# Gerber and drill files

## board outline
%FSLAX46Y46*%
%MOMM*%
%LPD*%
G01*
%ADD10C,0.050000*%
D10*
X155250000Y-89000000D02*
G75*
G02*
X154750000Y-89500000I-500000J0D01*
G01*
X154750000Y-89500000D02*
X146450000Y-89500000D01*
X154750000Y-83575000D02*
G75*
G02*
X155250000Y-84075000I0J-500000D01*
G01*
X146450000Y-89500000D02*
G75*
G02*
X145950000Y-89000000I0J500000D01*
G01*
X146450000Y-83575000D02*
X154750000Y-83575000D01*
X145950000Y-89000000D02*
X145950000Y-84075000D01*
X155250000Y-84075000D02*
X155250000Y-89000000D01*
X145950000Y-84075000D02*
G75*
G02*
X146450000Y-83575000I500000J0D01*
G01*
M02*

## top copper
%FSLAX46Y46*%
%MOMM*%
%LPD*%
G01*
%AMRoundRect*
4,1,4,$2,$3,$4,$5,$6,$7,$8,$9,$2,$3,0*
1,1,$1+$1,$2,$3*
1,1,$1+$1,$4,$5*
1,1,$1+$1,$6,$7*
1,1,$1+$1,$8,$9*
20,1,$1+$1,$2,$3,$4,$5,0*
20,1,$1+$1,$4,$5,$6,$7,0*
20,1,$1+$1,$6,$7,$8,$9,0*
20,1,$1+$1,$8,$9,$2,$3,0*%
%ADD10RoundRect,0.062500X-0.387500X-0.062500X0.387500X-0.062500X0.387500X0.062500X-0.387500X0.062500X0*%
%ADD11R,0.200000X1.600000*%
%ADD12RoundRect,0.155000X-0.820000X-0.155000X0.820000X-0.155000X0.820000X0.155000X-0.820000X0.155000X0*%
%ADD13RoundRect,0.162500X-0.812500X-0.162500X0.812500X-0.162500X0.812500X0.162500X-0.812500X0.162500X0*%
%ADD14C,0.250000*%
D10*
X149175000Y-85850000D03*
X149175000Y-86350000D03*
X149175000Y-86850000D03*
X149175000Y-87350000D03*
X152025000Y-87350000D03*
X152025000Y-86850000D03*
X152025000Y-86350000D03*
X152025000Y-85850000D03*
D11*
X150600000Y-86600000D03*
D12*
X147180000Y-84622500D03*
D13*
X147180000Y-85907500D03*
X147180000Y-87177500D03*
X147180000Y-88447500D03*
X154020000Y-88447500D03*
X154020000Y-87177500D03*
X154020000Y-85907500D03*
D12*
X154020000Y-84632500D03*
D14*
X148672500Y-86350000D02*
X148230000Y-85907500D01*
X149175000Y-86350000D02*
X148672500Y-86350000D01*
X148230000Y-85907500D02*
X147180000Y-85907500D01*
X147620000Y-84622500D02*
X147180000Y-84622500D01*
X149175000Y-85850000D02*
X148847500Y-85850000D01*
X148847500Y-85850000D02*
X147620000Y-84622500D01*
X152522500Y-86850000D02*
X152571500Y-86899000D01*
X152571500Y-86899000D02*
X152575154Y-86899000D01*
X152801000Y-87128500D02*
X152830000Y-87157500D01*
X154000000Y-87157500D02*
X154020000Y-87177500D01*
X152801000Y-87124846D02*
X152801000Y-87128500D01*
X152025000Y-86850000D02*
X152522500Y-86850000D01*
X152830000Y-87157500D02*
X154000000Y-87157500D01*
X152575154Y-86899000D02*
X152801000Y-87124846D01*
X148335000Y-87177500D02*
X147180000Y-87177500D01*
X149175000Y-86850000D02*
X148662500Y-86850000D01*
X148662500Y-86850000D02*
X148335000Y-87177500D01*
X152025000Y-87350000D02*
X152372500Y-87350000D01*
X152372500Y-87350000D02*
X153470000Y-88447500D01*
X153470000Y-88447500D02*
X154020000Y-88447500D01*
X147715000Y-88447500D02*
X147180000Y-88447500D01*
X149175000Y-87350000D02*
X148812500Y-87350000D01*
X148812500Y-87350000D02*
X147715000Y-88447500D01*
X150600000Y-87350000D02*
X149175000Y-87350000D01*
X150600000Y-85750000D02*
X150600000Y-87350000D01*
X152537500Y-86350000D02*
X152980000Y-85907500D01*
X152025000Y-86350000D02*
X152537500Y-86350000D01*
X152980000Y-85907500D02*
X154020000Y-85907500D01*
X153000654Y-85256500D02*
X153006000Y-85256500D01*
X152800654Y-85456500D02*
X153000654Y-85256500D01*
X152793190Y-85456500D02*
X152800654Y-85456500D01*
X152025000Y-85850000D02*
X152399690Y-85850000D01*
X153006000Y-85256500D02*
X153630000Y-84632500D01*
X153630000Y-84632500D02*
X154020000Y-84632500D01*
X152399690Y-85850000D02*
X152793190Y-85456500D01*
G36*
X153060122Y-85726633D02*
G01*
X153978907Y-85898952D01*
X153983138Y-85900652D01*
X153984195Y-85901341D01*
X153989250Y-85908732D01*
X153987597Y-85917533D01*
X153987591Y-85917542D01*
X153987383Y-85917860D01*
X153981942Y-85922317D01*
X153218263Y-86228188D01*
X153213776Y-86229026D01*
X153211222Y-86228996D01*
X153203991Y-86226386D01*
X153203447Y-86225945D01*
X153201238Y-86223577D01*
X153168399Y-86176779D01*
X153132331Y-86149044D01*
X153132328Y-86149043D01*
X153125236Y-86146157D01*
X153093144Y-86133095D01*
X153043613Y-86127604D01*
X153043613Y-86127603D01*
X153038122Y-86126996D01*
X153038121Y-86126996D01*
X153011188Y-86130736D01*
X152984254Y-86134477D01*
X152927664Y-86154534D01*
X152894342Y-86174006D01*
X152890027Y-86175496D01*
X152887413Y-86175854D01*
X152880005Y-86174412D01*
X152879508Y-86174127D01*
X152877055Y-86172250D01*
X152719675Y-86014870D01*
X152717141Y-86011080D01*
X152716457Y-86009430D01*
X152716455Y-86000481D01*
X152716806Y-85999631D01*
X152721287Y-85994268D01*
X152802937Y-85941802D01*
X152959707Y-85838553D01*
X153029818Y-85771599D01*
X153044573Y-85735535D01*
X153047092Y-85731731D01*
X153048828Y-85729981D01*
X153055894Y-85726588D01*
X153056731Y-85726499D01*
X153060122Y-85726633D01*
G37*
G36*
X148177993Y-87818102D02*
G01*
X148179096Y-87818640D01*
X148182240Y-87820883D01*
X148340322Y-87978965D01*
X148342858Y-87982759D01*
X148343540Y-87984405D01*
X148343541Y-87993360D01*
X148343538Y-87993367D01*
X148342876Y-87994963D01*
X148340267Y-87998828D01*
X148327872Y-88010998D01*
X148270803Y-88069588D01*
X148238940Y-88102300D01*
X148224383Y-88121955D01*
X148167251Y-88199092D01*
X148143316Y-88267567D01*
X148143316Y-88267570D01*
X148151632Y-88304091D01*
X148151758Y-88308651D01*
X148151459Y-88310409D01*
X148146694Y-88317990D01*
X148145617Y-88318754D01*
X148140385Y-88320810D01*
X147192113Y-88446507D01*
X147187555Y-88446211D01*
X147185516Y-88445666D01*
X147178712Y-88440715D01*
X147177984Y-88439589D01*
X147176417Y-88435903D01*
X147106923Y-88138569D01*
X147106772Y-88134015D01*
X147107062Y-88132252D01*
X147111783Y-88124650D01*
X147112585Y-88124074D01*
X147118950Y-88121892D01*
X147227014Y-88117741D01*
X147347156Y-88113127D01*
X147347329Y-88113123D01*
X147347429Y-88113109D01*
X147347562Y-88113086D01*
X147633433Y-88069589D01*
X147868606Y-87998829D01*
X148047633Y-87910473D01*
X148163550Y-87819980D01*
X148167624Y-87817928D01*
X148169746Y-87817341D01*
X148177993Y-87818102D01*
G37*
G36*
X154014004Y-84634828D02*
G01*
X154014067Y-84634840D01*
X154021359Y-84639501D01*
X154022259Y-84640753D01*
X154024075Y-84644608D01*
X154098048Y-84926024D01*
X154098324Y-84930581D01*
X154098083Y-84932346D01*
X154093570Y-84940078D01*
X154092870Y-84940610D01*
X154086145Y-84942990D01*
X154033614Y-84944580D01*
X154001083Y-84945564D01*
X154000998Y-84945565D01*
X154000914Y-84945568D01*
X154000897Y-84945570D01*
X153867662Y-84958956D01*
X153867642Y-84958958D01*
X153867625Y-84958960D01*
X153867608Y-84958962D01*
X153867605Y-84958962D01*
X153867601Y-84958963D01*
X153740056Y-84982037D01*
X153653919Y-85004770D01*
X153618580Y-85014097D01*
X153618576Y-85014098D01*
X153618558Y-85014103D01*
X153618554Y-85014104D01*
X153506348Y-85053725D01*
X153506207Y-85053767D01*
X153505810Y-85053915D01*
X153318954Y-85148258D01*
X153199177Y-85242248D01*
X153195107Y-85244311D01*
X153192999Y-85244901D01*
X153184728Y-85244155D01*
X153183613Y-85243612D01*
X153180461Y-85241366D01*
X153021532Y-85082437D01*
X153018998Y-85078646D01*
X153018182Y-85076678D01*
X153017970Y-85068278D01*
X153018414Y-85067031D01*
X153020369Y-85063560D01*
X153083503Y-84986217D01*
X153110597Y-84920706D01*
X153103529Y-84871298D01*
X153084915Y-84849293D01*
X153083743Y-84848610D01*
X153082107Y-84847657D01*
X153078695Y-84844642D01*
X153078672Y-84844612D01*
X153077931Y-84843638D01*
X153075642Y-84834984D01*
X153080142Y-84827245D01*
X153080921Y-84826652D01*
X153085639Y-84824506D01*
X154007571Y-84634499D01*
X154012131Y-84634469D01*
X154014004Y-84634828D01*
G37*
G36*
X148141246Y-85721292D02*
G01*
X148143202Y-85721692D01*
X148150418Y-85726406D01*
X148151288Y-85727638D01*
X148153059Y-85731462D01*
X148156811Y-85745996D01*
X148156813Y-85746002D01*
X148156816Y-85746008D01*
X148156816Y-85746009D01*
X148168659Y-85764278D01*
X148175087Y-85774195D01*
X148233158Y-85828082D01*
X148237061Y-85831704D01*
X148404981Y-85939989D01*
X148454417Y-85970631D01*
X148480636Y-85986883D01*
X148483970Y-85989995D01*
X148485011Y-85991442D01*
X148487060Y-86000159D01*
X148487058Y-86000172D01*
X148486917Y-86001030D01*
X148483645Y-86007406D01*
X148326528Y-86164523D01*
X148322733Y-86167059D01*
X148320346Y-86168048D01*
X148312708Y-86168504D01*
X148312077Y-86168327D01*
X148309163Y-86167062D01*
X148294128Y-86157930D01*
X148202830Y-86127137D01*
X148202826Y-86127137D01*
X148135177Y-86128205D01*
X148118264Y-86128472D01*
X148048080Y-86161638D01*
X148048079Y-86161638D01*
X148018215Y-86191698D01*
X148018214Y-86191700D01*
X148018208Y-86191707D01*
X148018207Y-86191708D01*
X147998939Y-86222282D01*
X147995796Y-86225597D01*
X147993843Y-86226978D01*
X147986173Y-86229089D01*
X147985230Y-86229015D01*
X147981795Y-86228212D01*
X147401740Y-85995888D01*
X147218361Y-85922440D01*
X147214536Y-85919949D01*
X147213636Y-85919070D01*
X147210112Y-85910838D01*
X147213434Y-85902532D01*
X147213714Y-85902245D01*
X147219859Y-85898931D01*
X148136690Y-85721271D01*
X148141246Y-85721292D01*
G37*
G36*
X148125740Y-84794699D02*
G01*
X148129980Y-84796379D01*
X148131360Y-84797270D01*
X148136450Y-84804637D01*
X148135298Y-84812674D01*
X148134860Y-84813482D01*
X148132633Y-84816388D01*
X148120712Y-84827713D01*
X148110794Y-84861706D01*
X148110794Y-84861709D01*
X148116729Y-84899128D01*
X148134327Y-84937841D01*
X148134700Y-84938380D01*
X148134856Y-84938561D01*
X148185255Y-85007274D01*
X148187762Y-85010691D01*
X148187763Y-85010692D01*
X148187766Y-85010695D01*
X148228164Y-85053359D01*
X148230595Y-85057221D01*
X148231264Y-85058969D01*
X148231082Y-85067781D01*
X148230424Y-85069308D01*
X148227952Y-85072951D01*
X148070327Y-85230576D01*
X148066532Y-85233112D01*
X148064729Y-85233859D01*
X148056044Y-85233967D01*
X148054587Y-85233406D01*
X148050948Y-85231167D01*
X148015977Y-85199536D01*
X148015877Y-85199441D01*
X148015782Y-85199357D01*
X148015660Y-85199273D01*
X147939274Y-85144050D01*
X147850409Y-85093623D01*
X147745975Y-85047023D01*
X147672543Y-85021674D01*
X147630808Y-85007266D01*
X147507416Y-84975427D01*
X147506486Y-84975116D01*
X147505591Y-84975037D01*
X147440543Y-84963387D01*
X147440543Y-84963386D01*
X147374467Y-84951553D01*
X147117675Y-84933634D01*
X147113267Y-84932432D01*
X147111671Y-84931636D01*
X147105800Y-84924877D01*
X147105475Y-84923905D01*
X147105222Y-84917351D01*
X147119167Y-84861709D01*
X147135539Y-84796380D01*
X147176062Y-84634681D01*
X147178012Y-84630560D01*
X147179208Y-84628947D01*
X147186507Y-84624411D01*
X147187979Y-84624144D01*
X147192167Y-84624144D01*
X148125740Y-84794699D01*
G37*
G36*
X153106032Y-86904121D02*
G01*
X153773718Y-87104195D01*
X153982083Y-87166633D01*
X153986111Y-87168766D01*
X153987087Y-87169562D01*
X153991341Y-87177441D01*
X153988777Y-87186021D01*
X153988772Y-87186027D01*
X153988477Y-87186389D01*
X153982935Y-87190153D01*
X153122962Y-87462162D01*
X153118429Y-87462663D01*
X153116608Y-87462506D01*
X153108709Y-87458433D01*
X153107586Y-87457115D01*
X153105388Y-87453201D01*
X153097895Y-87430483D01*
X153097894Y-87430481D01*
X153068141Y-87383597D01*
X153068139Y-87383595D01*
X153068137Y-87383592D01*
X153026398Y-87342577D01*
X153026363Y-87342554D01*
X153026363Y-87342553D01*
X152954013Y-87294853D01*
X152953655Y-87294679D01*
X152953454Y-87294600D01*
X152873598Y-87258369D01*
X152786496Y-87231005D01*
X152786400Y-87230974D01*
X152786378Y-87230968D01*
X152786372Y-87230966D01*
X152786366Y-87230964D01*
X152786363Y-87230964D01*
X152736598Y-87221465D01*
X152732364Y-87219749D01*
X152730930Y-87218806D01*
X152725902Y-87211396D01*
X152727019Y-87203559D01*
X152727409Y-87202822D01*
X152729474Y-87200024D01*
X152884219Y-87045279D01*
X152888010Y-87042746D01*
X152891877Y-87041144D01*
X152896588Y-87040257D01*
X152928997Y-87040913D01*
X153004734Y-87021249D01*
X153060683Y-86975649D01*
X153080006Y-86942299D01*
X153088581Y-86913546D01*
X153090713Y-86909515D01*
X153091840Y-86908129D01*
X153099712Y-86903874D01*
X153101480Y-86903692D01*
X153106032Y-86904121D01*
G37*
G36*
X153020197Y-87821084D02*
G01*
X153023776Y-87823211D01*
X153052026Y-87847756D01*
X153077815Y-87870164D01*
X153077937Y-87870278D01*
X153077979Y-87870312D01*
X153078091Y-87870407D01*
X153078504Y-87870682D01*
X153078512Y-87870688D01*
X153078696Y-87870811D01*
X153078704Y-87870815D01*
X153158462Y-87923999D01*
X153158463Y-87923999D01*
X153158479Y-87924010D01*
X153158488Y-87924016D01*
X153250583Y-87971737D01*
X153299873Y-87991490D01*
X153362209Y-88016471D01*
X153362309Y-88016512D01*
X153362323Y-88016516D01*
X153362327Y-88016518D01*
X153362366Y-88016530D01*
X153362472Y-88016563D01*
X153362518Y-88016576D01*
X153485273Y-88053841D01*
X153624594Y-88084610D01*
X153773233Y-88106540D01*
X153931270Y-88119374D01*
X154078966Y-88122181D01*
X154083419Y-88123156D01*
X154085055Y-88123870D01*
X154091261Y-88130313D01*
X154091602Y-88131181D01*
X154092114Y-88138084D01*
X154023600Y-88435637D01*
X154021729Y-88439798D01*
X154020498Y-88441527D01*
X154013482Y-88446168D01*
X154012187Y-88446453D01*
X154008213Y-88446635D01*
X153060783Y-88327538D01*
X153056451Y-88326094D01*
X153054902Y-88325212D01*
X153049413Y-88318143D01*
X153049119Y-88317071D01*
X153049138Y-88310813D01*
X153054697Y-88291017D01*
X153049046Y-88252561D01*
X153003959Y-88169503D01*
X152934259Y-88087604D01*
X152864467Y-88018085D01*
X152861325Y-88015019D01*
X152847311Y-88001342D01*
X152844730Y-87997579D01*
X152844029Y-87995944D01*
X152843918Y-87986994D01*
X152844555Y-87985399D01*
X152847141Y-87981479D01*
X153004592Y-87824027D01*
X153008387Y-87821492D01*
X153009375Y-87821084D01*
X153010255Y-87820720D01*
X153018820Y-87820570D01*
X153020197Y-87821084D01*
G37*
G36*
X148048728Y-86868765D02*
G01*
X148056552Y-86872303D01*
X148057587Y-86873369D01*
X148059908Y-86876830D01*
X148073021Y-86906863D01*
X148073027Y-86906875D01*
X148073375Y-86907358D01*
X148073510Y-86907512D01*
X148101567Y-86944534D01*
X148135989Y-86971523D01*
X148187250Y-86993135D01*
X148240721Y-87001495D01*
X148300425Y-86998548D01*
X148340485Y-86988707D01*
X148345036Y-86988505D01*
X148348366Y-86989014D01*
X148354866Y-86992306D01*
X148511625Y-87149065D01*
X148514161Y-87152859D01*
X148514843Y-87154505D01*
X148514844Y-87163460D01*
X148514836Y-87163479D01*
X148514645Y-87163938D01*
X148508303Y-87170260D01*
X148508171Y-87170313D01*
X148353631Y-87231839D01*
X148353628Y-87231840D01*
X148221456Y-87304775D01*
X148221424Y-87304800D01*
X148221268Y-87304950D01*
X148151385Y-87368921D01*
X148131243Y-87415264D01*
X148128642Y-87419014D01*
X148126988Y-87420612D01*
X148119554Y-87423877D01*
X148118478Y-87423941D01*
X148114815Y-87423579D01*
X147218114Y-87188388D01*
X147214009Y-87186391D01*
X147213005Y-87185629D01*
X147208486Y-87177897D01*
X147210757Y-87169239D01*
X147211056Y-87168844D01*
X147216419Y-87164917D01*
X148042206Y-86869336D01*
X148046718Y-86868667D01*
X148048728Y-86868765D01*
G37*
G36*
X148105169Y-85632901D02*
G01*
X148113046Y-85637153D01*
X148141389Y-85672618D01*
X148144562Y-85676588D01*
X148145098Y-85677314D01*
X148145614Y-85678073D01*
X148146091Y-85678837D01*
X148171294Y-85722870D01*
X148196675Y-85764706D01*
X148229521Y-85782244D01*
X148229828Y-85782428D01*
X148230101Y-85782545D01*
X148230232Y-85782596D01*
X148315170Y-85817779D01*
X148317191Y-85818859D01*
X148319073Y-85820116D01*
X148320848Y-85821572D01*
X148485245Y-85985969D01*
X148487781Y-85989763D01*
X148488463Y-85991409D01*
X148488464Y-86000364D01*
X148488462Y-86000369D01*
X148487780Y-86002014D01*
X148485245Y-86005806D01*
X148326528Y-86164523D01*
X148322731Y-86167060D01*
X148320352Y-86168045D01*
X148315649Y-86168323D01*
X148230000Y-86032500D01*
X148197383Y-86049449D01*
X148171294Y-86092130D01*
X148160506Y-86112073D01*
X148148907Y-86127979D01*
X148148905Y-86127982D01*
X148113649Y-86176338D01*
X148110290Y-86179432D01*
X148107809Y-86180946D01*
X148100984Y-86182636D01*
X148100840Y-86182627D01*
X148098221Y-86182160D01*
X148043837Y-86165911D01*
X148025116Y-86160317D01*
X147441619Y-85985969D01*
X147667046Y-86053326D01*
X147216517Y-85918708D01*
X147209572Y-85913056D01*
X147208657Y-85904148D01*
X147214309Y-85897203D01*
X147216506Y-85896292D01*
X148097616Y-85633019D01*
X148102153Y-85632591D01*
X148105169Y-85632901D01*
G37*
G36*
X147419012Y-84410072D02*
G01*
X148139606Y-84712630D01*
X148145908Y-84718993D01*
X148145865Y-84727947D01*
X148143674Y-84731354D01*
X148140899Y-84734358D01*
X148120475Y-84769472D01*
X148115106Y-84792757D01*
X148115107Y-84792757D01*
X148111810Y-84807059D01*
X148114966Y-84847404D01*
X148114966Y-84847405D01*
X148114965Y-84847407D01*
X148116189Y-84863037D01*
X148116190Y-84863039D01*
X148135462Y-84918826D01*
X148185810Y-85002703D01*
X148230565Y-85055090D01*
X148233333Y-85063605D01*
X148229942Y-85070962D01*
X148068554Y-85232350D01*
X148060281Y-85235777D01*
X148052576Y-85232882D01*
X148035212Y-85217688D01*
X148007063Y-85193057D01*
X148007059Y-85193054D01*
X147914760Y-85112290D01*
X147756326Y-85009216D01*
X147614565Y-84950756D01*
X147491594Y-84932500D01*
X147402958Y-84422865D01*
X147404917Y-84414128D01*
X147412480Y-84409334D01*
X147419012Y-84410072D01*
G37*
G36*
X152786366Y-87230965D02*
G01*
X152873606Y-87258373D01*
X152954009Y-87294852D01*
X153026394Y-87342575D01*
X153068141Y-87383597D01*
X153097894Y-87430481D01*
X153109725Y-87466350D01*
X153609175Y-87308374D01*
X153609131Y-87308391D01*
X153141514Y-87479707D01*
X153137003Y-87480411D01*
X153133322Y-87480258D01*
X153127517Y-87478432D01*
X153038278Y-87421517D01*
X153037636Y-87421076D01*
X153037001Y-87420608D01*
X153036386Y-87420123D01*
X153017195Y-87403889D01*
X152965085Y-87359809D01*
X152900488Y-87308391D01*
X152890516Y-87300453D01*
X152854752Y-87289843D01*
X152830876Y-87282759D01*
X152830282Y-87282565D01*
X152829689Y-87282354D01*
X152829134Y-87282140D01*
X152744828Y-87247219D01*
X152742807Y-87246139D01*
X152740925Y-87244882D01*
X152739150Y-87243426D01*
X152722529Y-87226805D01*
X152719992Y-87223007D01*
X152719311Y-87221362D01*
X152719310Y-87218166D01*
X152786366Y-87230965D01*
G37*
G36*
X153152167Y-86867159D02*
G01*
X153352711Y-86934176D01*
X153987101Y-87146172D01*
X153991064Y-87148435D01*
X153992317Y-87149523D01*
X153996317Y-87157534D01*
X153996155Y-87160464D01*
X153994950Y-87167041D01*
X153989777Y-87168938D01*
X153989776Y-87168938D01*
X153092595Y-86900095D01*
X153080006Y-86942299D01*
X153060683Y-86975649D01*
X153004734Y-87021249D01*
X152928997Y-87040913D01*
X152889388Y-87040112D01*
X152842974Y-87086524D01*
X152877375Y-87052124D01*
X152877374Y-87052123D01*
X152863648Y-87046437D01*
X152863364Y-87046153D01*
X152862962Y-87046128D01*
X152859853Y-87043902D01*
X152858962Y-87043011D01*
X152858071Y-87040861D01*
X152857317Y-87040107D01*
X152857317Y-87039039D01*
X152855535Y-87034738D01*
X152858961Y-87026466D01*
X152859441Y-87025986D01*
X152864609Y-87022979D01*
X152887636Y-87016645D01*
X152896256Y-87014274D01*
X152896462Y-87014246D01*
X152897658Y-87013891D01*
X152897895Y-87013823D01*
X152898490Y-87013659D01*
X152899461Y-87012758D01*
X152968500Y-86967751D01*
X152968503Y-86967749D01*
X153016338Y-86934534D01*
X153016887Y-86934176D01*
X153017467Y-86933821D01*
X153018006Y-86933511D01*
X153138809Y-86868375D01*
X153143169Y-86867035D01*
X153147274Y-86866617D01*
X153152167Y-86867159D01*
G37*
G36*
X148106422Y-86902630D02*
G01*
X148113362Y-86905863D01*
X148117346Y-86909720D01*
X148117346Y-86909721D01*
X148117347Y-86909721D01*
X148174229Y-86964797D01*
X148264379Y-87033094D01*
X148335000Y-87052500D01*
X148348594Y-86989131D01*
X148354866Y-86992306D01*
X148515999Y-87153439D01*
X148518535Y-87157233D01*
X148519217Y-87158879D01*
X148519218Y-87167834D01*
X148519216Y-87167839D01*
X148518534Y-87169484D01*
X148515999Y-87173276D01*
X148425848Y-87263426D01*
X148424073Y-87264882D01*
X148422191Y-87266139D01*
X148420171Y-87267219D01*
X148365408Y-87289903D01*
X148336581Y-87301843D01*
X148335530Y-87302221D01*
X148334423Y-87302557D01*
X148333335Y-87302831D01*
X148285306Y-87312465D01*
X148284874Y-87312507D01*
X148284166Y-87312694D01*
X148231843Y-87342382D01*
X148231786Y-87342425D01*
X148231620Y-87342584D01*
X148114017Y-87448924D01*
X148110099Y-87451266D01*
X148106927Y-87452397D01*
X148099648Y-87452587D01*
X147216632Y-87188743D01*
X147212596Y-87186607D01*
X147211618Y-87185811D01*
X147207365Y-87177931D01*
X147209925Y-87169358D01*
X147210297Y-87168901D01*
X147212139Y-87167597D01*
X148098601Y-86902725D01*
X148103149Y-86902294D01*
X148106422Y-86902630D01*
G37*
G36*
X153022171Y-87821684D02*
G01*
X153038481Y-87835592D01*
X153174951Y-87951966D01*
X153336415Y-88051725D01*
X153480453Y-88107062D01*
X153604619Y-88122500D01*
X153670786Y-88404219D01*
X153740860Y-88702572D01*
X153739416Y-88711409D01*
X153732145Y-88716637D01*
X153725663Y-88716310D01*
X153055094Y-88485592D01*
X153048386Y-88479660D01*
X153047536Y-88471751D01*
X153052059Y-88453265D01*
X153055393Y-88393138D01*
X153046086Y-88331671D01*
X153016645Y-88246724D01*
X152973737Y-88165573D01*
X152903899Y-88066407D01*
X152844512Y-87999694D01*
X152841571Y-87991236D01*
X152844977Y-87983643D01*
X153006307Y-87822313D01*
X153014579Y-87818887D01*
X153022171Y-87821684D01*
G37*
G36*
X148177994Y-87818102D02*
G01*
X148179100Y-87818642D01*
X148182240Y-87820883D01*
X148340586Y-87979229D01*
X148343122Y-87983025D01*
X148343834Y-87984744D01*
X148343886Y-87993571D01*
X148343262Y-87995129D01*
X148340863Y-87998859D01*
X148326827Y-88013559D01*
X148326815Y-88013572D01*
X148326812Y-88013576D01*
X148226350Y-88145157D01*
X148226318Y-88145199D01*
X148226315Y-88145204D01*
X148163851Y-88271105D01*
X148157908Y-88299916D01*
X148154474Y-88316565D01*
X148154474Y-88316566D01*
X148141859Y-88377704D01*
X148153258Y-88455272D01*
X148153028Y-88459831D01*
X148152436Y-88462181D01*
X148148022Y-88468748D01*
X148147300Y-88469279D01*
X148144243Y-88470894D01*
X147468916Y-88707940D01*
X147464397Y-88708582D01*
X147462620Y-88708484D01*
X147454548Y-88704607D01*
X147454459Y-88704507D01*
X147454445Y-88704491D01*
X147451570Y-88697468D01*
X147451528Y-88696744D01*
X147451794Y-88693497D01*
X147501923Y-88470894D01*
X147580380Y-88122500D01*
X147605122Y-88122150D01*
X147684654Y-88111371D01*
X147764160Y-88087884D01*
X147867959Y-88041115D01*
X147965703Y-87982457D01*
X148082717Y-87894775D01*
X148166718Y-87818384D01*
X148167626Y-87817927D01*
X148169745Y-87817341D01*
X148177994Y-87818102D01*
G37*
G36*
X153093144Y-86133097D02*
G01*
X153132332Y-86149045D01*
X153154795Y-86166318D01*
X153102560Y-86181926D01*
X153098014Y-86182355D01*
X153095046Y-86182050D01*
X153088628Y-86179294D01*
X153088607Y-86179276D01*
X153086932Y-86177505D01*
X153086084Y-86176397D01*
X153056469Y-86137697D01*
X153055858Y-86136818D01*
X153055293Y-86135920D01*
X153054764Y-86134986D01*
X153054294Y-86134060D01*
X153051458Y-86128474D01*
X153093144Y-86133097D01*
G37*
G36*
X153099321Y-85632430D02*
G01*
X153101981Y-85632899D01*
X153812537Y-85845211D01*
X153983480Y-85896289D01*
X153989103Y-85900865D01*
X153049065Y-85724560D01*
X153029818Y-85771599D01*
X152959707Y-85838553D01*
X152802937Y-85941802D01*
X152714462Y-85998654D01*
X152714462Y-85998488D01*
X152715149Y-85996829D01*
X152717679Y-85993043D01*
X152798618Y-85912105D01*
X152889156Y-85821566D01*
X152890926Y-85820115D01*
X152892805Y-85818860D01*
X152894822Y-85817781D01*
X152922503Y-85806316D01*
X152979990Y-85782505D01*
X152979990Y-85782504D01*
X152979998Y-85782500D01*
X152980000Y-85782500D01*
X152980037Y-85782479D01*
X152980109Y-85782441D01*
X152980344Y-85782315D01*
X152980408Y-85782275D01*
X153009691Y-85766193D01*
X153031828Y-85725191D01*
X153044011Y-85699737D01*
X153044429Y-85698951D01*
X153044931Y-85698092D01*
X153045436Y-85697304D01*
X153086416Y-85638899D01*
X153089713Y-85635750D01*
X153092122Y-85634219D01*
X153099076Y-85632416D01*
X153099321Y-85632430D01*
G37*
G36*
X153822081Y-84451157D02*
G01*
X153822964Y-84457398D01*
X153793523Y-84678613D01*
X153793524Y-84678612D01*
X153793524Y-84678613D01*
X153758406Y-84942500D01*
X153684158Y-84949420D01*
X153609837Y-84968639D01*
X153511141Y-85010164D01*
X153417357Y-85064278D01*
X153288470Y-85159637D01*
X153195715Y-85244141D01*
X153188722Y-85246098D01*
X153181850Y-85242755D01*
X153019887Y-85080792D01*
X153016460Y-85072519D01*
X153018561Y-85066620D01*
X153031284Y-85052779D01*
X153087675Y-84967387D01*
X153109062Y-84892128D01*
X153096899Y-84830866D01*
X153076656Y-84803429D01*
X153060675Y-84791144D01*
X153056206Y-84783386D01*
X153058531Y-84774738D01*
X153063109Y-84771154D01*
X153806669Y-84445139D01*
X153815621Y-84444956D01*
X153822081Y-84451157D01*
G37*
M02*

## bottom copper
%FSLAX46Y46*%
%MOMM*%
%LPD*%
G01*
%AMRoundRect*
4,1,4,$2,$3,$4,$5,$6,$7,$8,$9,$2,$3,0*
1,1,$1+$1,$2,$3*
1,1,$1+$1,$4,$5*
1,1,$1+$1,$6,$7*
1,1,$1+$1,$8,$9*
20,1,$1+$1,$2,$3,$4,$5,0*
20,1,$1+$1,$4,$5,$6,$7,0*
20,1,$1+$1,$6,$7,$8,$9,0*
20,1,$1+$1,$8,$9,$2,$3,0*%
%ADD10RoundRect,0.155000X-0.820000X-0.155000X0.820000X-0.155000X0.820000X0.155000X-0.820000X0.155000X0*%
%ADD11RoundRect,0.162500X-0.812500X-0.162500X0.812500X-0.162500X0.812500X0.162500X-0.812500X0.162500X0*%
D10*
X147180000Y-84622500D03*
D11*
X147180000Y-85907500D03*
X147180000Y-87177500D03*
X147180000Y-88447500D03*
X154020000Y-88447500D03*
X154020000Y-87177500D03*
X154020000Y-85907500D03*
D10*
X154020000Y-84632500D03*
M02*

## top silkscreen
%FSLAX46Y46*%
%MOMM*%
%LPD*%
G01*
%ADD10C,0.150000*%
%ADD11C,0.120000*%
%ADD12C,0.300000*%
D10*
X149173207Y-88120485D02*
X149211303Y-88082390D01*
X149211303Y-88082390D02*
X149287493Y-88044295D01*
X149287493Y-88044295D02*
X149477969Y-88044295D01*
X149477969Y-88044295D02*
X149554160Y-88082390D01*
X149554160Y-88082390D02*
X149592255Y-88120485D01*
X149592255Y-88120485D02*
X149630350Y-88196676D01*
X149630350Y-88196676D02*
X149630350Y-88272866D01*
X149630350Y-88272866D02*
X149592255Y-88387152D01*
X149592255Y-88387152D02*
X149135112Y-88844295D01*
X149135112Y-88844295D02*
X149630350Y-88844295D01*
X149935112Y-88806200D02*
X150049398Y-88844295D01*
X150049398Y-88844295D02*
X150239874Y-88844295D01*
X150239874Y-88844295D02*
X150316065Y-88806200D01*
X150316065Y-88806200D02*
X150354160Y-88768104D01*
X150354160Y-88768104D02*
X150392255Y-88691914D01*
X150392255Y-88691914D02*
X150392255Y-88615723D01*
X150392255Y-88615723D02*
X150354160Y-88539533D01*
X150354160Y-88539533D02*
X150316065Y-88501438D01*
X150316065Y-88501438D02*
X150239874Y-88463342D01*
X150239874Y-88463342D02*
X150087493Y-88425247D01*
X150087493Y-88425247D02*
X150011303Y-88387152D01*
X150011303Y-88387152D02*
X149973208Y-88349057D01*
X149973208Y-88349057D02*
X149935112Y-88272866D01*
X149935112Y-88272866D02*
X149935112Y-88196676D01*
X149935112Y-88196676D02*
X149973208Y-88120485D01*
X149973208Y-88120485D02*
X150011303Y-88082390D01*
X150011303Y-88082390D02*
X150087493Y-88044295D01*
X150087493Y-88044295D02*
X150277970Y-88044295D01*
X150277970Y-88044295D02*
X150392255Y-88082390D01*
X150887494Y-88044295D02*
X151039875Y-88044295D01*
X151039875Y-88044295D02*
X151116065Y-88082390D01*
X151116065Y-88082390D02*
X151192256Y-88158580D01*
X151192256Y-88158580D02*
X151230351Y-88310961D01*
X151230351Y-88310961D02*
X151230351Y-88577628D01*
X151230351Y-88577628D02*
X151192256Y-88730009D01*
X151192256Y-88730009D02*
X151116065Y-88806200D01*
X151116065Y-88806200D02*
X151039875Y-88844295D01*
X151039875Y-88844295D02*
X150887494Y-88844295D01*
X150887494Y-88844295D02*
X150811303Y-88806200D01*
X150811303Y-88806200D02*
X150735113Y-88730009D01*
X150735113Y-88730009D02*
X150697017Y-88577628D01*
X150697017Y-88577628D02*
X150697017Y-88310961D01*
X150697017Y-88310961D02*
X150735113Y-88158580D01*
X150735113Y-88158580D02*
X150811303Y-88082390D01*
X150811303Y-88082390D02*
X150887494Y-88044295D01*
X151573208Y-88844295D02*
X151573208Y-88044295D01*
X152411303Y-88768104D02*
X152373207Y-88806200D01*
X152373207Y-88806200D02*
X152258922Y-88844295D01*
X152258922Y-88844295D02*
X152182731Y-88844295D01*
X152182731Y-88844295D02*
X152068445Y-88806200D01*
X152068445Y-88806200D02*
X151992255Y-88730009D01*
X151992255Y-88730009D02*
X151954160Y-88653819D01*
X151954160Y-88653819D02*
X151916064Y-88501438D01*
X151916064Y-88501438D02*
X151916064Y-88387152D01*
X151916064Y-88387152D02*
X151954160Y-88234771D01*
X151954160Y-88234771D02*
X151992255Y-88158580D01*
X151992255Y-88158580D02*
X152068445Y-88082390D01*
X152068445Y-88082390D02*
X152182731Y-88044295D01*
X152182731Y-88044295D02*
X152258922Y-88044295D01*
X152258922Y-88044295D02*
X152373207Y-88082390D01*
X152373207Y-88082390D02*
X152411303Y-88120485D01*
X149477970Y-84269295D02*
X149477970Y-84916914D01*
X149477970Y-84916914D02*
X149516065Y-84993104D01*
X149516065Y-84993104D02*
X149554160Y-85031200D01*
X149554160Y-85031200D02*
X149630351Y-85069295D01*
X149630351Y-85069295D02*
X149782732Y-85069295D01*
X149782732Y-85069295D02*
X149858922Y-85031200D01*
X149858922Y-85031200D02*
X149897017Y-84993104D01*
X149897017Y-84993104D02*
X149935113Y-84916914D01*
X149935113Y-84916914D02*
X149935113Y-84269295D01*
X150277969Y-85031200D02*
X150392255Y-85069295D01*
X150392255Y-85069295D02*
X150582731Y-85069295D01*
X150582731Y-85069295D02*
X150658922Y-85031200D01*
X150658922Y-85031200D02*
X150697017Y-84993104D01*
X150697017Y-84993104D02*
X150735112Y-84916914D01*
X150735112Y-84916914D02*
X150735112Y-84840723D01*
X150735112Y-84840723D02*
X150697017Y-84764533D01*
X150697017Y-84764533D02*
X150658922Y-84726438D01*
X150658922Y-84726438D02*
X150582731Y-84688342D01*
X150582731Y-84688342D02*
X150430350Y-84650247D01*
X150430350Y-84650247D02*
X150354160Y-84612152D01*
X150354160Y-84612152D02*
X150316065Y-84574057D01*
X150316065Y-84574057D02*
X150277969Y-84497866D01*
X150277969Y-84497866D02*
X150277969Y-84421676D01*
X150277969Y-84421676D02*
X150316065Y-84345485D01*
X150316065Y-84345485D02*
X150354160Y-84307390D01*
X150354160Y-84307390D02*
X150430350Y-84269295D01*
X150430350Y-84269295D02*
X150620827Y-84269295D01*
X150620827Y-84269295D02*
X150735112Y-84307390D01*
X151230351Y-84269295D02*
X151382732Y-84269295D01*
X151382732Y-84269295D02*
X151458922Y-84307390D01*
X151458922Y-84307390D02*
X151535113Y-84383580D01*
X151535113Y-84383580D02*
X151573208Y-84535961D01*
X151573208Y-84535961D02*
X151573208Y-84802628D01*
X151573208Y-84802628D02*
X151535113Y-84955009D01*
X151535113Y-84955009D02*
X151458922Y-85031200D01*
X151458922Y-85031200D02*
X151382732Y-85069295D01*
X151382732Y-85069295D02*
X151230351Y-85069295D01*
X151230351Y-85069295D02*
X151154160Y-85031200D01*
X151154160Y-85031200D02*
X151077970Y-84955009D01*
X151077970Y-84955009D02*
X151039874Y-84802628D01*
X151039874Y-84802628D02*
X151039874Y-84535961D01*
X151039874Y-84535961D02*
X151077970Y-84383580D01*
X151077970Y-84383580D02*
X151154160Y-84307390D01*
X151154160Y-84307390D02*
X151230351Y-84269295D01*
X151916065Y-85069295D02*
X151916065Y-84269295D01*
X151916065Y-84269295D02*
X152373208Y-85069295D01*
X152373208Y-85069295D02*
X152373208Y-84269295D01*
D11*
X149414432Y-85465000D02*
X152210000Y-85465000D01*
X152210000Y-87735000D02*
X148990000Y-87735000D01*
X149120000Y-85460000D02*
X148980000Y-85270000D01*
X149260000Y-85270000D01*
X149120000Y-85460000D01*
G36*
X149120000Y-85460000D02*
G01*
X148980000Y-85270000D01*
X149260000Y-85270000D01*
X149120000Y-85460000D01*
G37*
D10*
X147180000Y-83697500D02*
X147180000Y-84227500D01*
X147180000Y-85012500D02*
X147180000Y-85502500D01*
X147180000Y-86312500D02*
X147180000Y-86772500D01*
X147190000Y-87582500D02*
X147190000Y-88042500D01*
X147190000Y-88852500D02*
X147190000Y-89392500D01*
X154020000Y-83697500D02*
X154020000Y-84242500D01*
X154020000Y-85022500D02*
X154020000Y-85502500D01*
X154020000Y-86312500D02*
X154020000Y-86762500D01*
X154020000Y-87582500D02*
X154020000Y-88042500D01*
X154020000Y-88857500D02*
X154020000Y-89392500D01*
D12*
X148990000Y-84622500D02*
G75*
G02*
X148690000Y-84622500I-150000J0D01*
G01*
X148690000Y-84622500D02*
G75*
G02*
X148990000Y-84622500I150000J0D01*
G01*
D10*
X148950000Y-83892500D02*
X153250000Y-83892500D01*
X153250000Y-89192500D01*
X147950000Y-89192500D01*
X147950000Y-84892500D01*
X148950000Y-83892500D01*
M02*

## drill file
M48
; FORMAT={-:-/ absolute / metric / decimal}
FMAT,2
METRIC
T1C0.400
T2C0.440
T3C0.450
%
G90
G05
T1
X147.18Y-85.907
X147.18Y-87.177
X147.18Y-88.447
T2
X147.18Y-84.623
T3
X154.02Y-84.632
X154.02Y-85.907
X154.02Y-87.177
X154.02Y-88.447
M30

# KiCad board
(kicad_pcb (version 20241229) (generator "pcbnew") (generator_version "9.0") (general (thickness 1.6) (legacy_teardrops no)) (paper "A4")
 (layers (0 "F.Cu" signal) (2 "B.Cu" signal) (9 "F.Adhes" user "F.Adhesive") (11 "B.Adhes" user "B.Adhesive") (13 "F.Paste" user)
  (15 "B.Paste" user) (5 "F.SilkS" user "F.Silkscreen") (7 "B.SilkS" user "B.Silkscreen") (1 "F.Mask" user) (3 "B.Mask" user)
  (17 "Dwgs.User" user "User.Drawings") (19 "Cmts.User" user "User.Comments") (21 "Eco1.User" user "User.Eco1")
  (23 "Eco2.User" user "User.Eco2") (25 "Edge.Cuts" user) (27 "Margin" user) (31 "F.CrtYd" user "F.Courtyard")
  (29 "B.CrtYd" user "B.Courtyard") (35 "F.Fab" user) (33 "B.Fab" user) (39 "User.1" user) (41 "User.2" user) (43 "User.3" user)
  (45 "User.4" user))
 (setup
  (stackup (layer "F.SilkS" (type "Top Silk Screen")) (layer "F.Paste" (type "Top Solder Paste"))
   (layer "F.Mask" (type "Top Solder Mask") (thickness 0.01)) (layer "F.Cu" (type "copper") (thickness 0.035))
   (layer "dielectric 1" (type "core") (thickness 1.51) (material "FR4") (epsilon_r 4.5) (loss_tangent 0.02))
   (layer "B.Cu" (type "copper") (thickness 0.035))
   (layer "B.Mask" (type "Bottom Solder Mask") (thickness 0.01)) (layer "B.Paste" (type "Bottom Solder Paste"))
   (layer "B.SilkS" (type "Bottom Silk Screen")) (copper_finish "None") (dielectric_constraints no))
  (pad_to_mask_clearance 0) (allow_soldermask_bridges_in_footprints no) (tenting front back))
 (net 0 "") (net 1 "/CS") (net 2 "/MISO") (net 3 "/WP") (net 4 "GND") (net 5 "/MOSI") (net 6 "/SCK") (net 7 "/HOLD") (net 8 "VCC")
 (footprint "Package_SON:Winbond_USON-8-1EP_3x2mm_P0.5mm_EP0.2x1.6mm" (layer "F.Cu") (at 150.6 86.6)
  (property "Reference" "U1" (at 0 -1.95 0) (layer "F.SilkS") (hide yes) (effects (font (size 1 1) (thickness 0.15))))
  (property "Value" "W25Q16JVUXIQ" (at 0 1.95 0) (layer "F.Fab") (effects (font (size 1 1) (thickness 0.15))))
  (fp_line (start -1.185568 -1.135) (end 1.61 -1.135) (stroke (width 0.12) (type solid)) (layer "F.SilkS"))
  (fp_line (start 1.61 1.135) (end -1.61 1.135) (stroke (width 0.12) (type solid)) (layer "F.SilkS"))
  (fp_poly (pts (xy -1.48 -1.14) (xy -1.62 -1.33) (xy -1.34 -1.33)) (stroke (width 0.12) (type solid)) (fill yes) (layer "F.SilkS"))
  (pad "" smd roundrect (at 0 0) (size 0.16 1.29) (layers "F.Paste") (roundrect_rratio 0.25)
   (teardrops (best_length_ratio 0.5) (max_length 1) (best_width_ratio 1) (max_width 2) (curved_edges yes) (filter_ratio 0.9) (enabled yes)
    (allow_two_segments yes) (prefer_zone_connections yes)))
  (pad "1" smd roundrect (at -1.425 -0.75) (size 0.9 0.25) (layers "F.Cu" "F.Mask" "F.Paste") (roundrect_rratio 0.25) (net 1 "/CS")
   (teardrops (best_length_ratio 0.5) (max_length 1) (best_width_ratio 1) (max_width 2) (curved_edges yes) (filter_ratio 0.9) (enabled yes)
    (allow_two_segments yes) (prefer_zone_connections yes)))
  (pad "2" smd roundrect (at -1.425 -0.25) (size 0.9 0.25) (layers "F.Cu" "F.Mask" "F.Paste") (roundrect_rratio 0.25) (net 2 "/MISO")
   (teardrops (best_length_ratio 0.5) (max_length 1) (best_width_ratio 1) (max_width 2) (curved_edges yes) (filter_ratio 0.9) (enabled yes)
    (allow_two_segments yes) (prefer_zone_connections yes)))
  (pad "3" smd roundrect (at -1.425 0.25) (size 0.9 0.25) (layers "F.Cu" "F.Mask" "F.Paste") (roundrect_rratio 0.25) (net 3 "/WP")
   (teardrops (best_length_ratio 0.5) (max_length 1) (best_width_ratio 1) (max_width 2) (curved_edges yes) (filter_ratio 0.9) (enabled yes)
    (allow_two_segments yes) (prefer_zone_connections yes)))
  (pad "4" smd roundrect (at -1.425 0.75) (size 0.9 0.25) (layers "F.Cu" "F.Mask" "F.Paste") (roundrect_rratio 0.25) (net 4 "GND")
   (teardrops (best_length_ratio 0.5) (max_length 1) (best_width_ratio 1) (max_width 2) (curved_edges yes) (filter_ratio 0.9) (enabled yes)
    (allow_two_segments yes) (prefer_zone_connections yes)))
  (pad "5" smd roundrect (at 1.425 0.75) (size 0.9 0.25) (layers "F.Cu" "F.Mask" "F.Paste") (roundrect_rratio 0.25) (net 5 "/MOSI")
   (teardrops (best_length_ratio 0.5) (max_length 1) (best_width_ratio 1) (max_width 2) (curved_edges yes) (filter_ratio 0.9) (enabled yes)
    (allow_two_segments yes) (prefer_zone_connections yes)))
  (pad "6" smd roundrect (at 1.425 0.25) (size 0.9 0.25) (layers "F.Cu" "F.Mask" "F.Paste") (roundrect_rratio 0.25) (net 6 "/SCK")
   (teardrops (best_length_ratio 0.5) (max_length 1) (best_width_ratio 1) (max_width 2) (curved_edges yes) (filter_ratio 0.9) (enabled yes)
    (allow_two_segments yes) (prefer_zone_connections yes)))
  (pad "7" smd roundrect (at 1.425 -0.25) (size 0.9 0.25) (layers "F.Cu" "F.Mask" "F.Paste") (roundrect_rratio 0.25) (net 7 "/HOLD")
   (teardrops (best_length_ratio 0.5) (max_length 1) (best_width_ratio 1) (max_width 2) (curved_edges yes) (filter_ratio 0.9) (enabled yes)
    (allow_two_segments yes) (prefer_zone_connections yes)))
  (pad "8" smd roundrect (at 1.425 -0.75) (size 0.9 0.25) (layers "F.Cu" "F.Mask" "F.Paste") (roundrect_rratio 0.25) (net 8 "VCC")
   (teardrops (best_length_ratio 0.5) (max_length 1) (best_width_ratio 1) (max_width 2) (curved_edges yes) (filter_ratio 0.9) (enabled yes)
    (allow_two_segments yes) (prefer_zone_connections yes)))
  (pad "9" smd rect (at 0 0) (size 0.2 1.6) (layers "F.Cu" "F.Mask") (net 4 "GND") (zone_connect 2)
   (teardrops (best_length_ratio 0.5) (max_length 1) (best_width_ratio 1) (max_width 2) (curved_edges yes) (filter_ratio 0.9) (enabled yes)
    (allow_two_segments yes) (prefer_zone_connections yes))))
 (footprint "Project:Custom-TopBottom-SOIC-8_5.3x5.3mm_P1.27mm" (layer "F.Cu") (at 150.6 86.5425)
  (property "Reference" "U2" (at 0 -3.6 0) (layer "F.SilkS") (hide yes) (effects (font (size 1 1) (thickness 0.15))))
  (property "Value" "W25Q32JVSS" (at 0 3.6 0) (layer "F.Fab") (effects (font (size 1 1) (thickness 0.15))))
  (fp_line (start -3.42 -2.845) (end -3.42 -2.315) (stroke (width 0.15) (type default)) (layer "F.SilkS"))
  (fp_line (start -3.42 -1.53) (end -3.42 -1.04) (stroke (width 0.15) (type default)) (layer "F.SilkS"))
  (fp_line (start -3.42 -0.23) (end -3.42 0.23) (stroke (width 0.15) (type default)) (layer "F.SilkS"))
  (fp_line (start -3.41 1.04) (end -3.41 1.5) (stroke (width 0.15) (type default)) (layer "F.SilkS"))
  (fp_line (start -3.41 2.31) (end -3.41 2.85) (stroke (width 0.15) (type default)) (layer "F.SilkS"))
  (fp_line (start 3.42 -2.845) (end 3.42 -2.3) (stroke (width 0.15) (type default)) (layer "F.SilkS"))
  (fp_line (start 3.42 -1.52) (end 3.42 -1.04) (stroke (width 0.15) (type default)) (layer "F.SilkS"))
  (fp_line (start 3.42 -0.23) (end 3.42 0.22) (stroke (width 0.15) (type default)) (layer "F.SilkS"))
  (fp_line (start 3.42 1.04) (end 3.42 1.5) (stroke (width 0.15) (type default)) (layer "F.SilkS"))
  (fp_line (start 3.42 2.315) (end 3.42 2.85) (stroke (width 0.15) (type default)) (layer "F.SilkS"))
  (fp_circle (center -1.76 -1.92) (end -1.51 -1.92) (stroke (width 0.1) (type default)) (fill yes) (layer "F.SilkS"))
  (fp_poly
   (pts (xy -1.65 -2.65) (xy 2.65 -2.65) (xy 2.65 2.65) (xy -2.65 2.65) (xy -2.65 -1.65)) (stroke (width 0.15) (type solid)) (fill no)
   (layer "F.SilkS"))
  (pad "1" thru_hole roundrect (at -3.42 -1.92) (size 1.95 0.62) (drill 0.44) (layers "*.Cu" "*.Mask") (remove_unused_layers no)
   (roundrect_rratio 0.25) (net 1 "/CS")
   (teardrops (best_length_ratio 0.5) (max_length 1) (best_width_ratio 1) (max_width 2) (curved_edges yes) (filter_ratio 0.9) (enabled yes)
    (allow_two_segments yes) (prefer_zone_connections yes)))
  (pad "2" thru_hole roundrect (at -3.42 -0.635) (size 1.95 0.65) (drill 0.4) (layers "*.Cu" "*.Mask") (remove_unused_layers no)
   (roundrect_rratio 0.25) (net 2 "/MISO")
   (teardrops (best_length_ratio 0.5) (max_length 1) (best_width_ratio 1) (max_width 2) (curved_edges yes) (filter_ratio 0.9) (enabled yes)
    (allow_two_segments yes) (prefer_zone_connections yes)))
  (pad "3" thru_hole roundrect (at -3.42 0.635) (size 1.95 0.65) (drill 0.4) (layers "*.Cu" "*.Mask") (remove_unused_layers no)
   (roundrect_rratio 0.25) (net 3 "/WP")
   (teardrops (best_length_ratio 0.5) (max_length 1) (best_width_ratio 1) (max_width 2) (curved_edges yes) (filter_ratio 0.9) (enabled yes)
    (allow_two_segments yes) (prefer_zone_connections yes)))
  (pad "4" thru_hole roundrect (at -3.42 1.905) (size 1.95 0.65) (drill 0.4) (layers "*.Cu" "*.Mask") (remove_unused_layers no)
   (roundrect_rratio 0.25) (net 4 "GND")
   (teardrops (best_length_ratio 0.5) (max_length 1) (best_width_ratio 1) (max_width 2) (curved_edges yes) (filter_ratio 0.9) (enabled yes)
    (allow_two_segments yes) (prefer_zone_connections yes)))
  (pad "5" thru_hole roundrect (at 3.42 1.905) (size 1.95 0.65) (drill 0.45) (layers "*.Cu" "*.Mask") (remove_unused_layers no)
   (roundrect_rratio 0.25) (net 5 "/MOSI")
   (teardrops (best_length_ratio 0.5) (max_length 1) (best_width_ratio 1) (max_width 2) (curved_edges yes) (filter_ratio 0.9) (enabled yes)
    (allow_two_segments yes) (prefer_zone_connections yes)))
  (pad "6" thru_hole roundrect (at 3.42 0.635) (size 1.95 0.65) (drill 0.45) (layers "*.Cu" "*.Mask") (remove_unused_layers no)
   (roundrect_rratio 0.25) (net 6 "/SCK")
   (teardrops (best_length_ratio 0.5) (max_length 1) (best_width_ratio 1) (max_width 2) (curved_edges yes) (filter_ratio 0.9) (enabled yes)
    (allow_two_segments yes) (prefer_zone_connections yes)))
  (pad "7" thru_hole roundrect (at 3.42 -0.635) (size 1.95 0.65) (drill 0.45) (layers "*.Cu" "*.Mask") (remove_unused_layers no)
   (roundrect_rratio 0.25) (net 7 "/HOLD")
   (teardrops (best_length_ratio 0.5) (max_length 1) (best_width_ratio 1) (max_width 2) (curved_edges yes) (filter_ratio 0.9) (enabled yes)
    (allow_two_segments yes) (prefer_zone_connections yes)))
  (pad "8" thru_hole roundrect (at 3.42 -1.91) (size 1.95 0.62) (drill 0.45) (layers "*.Cu" "*.Mask") (remove_unused_layers no)
   (roundrect_rratio 0.25) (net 8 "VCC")
   (teardrops (best_length_ratio 0.5) (max_length 1) (best_width_ratio 1) (max_width 2) (curved_edges yes) (filter_ratio 0.9) (enabled yes)
    (allow_two_segments yes) (prefer_zone_connections yes))))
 (gr_arc (start 155.25 89) (mid 155.103553 89.353553) (end 154.75 89.5) (stroke (width 0.05) (type default)) (layer "Edge.Cuts"))
 (gr_line (start 154.75 89.5) (end 146.45 89.5) (stroke (width 0.05) (type default)) (layer "Edge.Cuts"))
 (gr_arc (start 154.75 83.575) (mid 155.103553 83.721447) (end 155.25 84.075) (stroke (width 0.05) (type default)) (layer "Edge.Cuts"))
 (gr_arc (start 146.45 89.5) (mid 146.096447 89.353553) (end 145.95 89) (stroke (width 0.05) (type default)) (layer "Edge.Cuts"))
 (gr_line (start 146.45 83.575) (end 154.75 83.575) (stroke (width 0.05) (type default)) (layer "Edge.Cuts"))
 (gr_line (start 145.95 89) (end 145.95 84.075) (stroke (width 0.05) (type default)) (layer "Edge.Cuts"))
 (gr_line (start 155.25 84.075) (end 155.25 89) (stroke (width 0.05) (type default)) (layer "Edge.Cuts"))
 (gr_arc (start 145.95 84.075) (mid 146.096447 83.721447) (end 146.45 83.575) (stroke (width 0.05) (type default)) (layer "Edge.Cuts"))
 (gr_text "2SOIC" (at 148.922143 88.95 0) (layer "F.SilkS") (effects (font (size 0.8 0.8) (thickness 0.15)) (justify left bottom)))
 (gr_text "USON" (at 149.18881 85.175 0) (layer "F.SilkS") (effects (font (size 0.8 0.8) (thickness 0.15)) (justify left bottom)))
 (segment (start 148.6725 86.35) (end 148.23 85.9075) (width 0.25) (layer "F.Cu") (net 2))
 (segment (start 149.175 86.35) (end 148.6725 86.35) (width 0.25) (layer "F.Cu") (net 2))
 (segment (start 148.23 85.9075) (end 147.18 85.9075) (width 0.25) (layer "F.Cu") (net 2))
 (segment (start 147.62 84.6225) (end 147.18 84.6225) (width 0.25) (layer "F.Cu") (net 1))
 (segment (start 149.175 85.85) (end 148.8475 85.85) (width 0.25) (layer "F.Cu") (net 1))
 (segment (start 148.8475 85.85) (end 147.62 84.6225) (width 0.25) (layer "F.Cu") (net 1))
 (segment (start 152.5225 86.85) (end 152.5715 86.899) (width 0.25) (layer "F.Cu") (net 6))
 (segment (start 152.5715 86.899) (end 152.575154 86.899) (width 0.25) (layer "F.Cu") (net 6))
 (segment (start 152.801 87.1285) (end 152.83 87.1575) (width 0.25) (layer "F.Cu") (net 6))
 (segment (start 154 87.1575) (end 154.02 87.1775) (width 0.25) (layer "F.Cu") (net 6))
 (segment (start 152.801 87.124846) (end 152.801 87.1285) (width 0.25) (layer "F.Cu") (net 6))
 (segment (start 152.025 86.85) (end 152.5225 86.85) (width 0.25) (layer "F.Cu") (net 6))
 (segment (start 152.83 87.1575) (end 154 87.1575) (width 0.25) (layer "F.Cu") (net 6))
 (segment (start 152.575154 86.899) (end 152.801 87.124846) (width 0.25) (layer "F.Cu") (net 6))
 (segment (start 148.335 87.1775) (end 147.18 87.1775) (width 0.25) (layer "F.Cu") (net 3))
 (segment (start 149.175 86.85) (end 148.6625 86.85) (width 0.25) (layer "F.Cu") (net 3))
 (segment (start 148.6625 86.85) (end 148.335 87.1775) (width 0.25) (layer "F.Cu") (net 3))
 (segment (start 152.025 87.35) (end 152.3725 87.35) (width 0.25) (layer "F.Cu") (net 5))
 (segment (start 152.3725 87.35) (end 153.47 88.4475) (width 0.25) (layer "F.Cu") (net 5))
 (segment (start 153.47 88.4475) (end 154.02 88.4475) (width 0.25) (layer "F.Cu") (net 5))
 (segment (start 147.715 88.4475) (end 147.18 88.4475) (width 0.25) (layer "F.Cu") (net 4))
 (segment (start 149.175 87.35) (end 148.8125 87.35) (width 0.25) (layer "F.Cu") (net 4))
 (segment (start 148.8125 87.35) (end 147.715 88.4475) (width 0.25) (layer "F.Cu") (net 4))
 (segment (start 150.6 87.35) (end 149.175 87.35) (width 0.25) (layer "F.Cu") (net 4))
 (segment (start 150.6 85.75) (end 150.6 87.35) (width 0.25) (layer "F.Cu") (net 4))
 (segment (start 152.5375 86.35) (end 152.98 85.9075) (width 0.25) (layer "F.Cu") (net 7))
 (segment (start 152.025 86.35) (end 152.5375 86.35) (width 0.25) (layer "F.Cu") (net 7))
 (segment (start 152.98 85.9075) (end 154.02 85.9075) (width 0.25) (layer "F.Cu") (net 7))
 (segment (start 153.000654 85.2565) (end 153.006 85.2565) (width 0.25) (layer "F.Cu") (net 8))
 (segment (start 152.800654 85.4565) (end 153.000654 85.2565) (width 0.25) (layer "F.Cu") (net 8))
 (segment (start 152.79319 85.4565) (end 152.800654 85.4565) (width 0.25) (layer "F.Cu") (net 8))
 (segment (start 152.025 85.85) (end 152.39969 85.85) (width 0.25) (layer "F.Cu") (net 8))
 (segment (start 153.006 85.2565) (end 153.63 84.6325) (width 0.25) (layer "F.Cu") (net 8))
 (segment (start 153.63 84.6325) (end 154.02 84.6325) (width 0.25) (layer "F.Cu") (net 8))
 (segment (start 152.39969 85.85) (end 152.79319 85.4565) (width 0.25) (layer "F.Cu") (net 8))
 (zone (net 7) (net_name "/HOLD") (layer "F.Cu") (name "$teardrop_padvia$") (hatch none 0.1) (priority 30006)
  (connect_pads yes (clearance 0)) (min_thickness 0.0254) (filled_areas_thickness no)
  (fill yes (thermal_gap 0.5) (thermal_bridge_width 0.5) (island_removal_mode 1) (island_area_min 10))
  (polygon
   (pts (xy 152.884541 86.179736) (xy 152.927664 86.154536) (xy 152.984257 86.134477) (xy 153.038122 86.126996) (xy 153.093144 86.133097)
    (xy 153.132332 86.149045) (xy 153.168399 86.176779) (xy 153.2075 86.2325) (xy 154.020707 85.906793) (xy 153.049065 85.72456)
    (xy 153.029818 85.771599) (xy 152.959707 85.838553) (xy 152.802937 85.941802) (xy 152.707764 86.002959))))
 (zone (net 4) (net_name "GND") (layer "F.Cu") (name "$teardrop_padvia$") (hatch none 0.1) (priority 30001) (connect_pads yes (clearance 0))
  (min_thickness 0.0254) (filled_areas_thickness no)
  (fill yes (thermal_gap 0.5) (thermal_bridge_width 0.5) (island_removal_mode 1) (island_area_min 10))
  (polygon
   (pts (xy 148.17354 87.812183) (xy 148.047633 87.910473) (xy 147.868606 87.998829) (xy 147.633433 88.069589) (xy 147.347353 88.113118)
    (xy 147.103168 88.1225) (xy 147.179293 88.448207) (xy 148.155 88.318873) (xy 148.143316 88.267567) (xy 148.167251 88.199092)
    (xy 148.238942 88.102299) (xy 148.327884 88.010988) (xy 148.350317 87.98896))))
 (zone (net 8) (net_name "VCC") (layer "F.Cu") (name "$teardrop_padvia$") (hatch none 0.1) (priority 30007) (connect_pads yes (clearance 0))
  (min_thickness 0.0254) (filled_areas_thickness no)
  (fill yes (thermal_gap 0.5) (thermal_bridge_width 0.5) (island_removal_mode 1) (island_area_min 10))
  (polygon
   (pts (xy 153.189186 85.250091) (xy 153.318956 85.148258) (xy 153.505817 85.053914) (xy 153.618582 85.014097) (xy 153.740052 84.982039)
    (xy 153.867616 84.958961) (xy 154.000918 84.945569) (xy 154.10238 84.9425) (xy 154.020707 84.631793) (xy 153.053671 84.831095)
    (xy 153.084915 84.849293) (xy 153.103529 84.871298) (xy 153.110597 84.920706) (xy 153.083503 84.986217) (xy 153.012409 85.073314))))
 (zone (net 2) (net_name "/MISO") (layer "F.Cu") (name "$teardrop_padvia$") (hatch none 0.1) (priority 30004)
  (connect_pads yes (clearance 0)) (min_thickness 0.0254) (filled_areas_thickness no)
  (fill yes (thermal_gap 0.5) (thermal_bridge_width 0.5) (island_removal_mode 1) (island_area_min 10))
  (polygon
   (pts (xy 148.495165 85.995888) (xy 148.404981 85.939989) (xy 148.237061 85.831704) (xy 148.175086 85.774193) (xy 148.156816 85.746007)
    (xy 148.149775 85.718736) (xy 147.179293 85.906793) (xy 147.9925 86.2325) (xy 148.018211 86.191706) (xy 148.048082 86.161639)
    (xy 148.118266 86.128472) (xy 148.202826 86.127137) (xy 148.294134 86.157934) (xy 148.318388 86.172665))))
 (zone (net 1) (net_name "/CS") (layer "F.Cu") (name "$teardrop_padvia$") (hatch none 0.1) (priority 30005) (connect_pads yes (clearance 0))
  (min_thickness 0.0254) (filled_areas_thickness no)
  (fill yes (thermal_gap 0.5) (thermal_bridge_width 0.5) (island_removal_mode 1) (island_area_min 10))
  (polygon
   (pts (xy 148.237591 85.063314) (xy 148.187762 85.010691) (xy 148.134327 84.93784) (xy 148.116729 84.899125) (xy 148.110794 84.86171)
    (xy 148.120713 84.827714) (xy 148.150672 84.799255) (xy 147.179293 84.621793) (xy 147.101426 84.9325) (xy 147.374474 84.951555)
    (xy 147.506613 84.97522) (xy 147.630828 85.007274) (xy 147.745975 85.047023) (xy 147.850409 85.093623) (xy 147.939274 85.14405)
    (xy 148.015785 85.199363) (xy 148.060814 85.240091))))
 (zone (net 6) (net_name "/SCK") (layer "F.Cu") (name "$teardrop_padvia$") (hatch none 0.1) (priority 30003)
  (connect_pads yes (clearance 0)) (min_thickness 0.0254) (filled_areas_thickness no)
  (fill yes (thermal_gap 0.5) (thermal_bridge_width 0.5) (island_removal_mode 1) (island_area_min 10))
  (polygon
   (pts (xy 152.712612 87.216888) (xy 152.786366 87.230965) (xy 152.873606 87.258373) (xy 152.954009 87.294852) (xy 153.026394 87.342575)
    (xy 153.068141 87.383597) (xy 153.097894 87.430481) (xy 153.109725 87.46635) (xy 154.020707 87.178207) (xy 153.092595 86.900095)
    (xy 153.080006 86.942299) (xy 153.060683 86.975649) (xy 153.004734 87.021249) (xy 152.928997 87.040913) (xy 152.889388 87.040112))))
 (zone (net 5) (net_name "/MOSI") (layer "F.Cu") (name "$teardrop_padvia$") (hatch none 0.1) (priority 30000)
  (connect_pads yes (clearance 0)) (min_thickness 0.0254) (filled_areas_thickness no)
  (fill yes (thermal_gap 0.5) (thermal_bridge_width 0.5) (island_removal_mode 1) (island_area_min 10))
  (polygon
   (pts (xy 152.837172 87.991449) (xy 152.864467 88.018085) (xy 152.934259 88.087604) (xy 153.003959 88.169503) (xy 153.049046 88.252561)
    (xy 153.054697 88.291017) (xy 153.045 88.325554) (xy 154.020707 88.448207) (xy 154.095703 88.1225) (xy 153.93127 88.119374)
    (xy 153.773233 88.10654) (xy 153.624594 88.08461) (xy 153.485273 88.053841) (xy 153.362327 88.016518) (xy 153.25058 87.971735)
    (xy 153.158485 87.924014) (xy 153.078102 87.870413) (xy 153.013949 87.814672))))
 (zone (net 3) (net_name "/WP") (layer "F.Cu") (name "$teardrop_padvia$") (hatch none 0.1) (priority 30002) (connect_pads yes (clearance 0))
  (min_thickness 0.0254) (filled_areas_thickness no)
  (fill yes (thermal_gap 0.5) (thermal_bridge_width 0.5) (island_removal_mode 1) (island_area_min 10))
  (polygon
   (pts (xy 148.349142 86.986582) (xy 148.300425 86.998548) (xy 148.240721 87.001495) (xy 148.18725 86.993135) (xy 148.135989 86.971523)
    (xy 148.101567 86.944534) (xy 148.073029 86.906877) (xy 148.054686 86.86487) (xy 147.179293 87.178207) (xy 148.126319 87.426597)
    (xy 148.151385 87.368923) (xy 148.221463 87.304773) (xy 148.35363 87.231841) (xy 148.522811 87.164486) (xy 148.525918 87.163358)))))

